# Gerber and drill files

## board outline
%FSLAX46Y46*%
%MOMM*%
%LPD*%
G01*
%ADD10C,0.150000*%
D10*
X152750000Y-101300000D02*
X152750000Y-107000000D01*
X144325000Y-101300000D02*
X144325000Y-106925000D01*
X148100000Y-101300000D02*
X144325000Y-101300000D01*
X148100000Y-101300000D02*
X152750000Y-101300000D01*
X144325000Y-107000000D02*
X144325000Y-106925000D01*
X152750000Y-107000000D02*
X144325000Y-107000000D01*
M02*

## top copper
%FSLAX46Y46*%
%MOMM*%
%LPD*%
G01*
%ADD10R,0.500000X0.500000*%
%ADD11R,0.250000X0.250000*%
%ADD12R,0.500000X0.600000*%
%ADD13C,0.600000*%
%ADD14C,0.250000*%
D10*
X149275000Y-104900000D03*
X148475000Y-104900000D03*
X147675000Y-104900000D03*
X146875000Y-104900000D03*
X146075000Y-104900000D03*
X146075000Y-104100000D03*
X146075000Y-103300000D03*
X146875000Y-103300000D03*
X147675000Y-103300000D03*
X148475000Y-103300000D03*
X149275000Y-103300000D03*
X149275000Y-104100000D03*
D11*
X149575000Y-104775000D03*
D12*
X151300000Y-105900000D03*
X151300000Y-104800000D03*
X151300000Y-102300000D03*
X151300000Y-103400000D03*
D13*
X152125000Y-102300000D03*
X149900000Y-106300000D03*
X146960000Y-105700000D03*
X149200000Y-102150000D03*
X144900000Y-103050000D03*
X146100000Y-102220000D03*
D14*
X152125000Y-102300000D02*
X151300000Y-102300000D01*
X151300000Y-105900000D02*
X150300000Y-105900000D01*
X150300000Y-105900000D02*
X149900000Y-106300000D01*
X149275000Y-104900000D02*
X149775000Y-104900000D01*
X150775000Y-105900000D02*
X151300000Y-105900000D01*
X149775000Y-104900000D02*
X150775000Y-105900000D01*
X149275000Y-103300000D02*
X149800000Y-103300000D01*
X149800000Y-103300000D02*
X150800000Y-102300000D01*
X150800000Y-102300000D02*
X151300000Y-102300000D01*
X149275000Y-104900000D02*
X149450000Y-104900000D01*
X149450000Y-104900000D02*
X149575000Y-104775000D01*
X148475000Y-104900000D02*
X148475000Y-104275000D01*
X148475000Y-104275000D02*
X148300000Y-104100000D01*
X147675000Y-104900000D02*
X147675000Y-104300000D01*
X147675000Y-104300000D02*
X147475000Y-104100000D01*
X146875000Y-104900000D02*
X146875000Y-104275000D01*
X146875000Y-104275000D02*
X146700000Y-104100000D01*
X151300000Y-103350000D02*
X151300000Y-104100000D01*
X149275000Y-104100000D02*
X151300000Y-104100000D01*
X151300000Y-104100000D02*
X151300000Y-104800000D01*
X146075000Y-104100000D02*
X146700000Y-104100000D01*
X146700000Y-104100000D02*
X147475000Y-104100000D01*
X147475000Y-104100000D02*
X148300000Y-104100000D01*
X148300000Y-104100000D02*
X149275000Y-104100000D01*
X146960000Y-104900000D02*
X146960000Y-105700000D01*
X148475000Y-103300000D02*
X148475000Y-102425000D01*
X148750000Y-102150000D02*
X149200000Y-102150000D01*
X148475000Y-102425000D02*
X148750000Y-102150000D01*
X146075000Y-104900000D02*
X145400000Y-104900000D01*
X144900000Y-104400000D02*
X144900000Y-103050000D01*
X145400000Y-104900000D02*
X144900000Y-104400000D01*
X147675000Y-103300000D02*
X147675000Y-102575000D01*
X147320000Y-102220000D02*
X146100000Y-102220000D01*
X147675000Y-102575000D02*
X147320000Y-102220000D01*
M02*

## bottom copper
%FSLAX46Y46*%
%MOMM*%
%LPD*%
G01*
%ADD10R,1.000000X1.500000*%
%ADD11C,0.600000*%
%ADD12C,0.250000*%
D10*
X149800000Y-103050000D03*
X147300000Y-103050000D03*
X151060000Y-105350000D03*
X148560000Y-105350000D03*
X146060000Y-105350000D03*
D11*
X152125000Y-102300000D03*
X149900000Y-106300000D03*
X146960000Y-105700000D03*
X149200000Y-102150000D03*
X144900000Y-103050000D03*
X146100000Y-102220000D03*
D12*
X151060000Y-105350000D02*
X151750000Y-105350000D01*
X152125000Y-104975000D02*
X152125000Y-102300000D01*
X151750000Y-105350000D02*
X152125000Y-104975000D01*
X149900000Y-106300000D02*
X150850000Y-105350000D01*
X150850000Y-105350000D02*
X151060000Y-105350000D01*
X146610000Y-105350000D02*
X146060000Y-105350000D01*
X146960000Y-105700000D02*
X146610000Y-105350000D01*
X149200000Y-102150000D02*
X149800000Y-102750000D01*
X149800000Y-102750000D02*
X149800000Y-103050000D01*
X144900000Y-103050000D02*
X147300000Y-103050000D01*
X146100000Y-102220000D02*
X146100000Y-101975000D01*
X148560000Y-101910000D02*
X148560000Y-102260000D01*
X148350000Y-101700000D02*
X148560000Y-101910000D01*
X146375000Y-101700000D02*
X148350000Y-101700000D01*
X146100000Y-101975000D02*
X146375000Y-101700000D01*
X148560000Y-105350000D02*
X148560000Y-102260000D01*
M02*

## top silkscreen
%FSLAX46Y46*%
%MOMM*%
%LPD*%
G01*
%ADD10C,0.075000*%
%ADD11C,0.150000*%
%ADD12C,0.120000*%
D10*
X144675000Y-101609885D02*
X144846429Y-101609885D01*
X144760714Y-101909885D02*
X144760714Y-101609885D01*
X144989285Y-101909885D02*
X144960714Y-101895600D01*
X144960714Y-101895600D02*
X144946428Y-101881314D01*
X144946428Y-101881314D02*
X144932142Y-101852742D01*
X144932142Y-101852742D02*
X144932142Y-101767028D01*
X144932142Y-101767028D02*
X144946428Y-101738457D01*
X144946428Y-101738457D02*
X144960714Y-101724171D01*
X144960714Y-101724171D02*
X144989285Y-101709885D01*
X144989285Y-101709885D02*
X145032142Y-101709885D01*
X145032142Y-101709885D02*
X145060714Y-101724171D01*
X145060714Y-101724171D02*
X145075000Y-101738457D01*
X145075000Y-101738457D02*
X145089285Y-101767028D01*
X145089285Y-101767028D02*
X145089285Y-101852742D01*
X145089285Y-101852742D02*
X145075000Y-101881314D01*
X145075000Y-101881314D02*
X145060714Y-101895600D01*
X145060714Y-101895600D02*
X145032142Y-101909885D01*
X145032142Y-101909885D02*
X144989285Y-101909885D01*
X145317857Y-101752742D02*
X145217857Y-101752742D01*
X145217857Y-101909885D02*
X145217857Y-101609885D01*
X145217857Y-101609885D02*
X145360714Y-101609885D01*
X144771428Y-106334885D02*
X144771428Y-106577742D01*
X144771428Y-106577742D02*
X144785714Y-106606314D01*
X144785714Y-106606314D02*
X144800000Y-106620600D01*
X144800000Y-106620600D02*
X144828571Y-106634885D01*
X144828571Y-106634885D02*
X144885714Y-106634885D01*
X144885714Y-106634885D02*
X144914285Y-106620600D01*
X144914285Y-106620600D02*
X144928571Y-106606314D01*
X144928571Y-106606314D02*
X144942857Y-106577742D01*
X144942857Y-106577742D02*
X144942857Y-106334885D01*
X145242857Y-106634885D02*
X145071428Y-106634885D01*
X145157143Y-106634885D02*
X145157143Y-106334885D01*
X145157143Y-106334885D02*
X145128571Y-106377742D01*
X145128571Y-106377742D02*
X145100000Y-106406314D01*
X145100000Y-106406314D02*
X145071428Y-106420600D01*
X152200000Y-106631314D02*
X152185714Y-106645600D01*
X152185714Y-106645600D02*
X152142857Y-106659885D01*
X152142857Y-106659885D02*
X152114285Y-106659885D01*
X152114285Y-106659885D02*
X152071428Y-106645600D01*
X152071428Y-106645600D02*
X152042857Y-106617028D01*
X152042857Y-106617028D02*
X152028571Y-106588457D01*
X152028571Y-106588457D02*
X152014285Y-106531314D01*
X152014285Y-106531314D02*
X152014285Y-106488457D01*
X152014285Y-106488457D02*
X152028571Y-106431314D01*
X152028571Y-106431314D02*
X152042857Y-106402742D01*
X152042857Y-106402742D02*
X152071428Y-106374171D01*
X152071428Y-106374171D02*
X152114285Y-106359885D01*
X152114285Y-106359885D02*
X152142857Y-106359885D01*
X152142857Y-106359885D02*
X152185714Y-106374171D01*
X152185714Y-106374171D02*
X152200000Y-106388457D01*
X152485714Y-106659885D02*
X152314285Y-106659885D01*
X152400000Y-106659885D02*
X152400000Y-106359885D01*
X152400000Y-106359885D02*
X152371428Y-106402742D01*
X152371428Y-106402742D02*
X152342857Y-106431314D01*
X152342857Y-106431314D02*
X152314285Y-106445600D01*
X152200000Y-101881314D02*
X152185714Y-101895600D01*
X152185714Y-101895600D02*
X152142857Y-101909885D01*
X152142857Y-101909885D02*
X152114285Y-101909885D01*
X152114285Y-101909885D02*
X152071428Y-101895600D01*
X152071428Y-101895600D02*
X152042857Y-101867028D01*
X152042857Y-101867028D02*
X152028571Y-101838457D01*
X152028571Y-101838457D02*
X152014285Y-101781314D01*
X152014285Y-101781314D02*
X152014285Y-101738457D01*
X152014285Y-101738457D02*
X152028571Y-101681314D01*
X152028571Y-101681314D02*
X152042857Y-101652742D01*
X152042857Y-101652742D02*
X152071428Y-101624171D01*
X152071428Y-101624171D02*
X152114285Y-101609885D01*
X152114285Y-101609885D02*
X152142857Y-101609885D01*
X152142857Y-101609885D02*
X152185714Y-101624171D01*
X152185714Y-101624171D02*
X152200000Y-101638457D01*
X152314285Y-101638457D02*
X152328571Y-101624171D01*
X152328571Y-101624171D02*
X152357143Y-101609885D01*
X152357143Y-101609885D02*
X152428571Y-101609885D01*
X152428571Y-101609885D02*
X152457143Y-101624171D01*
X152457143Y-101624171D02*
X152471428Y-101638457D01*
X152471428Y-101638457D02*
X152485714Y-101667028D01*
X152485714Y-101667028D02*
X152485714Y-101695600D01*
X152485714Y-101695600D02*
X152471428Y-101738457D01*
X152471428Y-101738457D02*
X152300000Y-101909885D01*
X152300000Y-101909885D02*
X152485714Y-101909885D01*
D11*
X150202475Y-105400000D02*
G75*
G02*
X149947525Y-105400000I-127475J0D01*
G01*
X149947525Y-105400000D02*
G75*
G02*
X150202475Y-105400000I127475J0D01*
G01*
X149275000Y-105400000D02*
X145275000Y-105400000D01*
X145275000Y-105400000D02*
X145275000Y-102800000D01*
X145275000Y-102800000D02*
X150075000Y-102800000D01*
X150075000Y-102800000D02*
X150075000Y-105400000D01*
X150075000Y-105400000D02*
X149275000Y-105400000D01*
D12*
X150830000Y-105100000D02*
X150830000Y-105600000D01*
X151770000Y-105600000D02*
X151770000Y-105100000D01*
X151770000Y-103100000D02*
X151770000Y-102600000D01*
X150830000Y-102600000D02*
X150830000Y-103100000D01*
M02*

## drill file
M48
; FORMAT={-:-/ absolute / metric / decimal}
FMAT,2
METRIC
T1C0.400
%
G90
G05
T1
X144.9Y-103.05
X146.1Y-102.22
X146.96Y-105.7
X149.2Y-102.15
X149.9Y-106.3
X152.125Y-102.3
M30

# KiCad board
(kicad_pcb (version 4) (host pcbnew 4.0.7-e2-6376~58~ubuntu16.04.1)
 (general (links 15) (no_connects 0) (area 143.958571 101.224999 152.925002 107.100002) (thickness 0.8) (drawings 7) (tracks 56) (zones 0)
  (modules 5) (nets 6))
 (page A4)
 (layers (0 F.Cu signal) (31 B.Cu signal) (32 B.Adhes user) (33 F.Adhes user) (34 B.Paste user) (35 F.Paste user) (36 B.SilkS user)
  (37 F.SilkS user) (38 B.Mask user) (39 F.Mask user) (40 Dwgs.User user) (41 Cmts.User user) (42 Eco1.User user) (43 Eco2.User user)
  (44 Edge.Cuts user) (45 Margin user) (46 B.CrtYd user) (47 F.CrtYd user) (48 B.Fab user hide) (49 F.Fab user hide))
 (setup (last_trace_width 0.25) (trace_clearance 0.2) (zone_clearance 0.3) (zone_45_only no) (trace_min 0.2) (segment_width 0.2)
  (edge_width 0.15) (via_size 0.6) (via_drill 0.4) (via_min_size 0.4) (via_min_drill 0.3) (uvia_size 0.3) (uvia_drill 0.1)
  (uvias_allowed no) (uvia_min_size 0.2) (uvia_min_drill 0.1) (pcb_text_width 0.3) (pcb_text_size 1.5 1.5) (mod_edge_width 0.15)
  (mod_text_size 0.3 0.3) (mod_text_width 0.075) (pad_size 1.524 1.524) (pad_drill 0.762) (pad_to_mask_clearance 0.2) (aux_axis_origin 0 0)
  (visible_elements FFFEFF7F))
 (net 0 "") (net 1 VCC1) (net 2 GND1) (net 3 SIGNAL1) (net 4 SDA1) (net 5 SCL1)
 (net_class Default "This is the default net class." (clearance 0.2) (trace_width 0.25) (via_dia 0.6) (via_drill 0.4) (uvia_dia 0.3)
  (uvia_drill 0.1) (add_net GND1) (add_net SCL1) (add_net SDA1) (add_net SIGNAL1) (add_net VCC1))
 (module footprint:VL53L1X (layer F.Cu) (at 149.275 104.9 90)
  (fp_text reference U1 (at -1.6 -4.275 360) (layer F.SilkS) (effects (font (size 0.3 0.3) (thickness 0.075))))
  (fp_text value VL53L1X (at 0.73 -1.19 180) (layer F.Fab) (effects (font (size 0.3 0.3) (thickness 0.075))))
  (fp_circle (center -0.5 0.8) (end -0.375 0.825) (layer F.SilkS) (width 0.15))
  (fp_line (start -0.5 0) (end -0.5 -4) (layer F.SilkS) (width 0.15))
  (fp_line (start -0.5 -4) (end 2.1 -4) (layer F.SilkS) (width 0.15))
  (fp_line (start 2.1 -4) (end 2.1 0.8) (layer F.SilkS) (width 0.15))
  (fp_line (start 2.1 0.8) (end -0.5 0.8) (layer F.SilkS) (width 0.15))
  (fp_line (start -0.5 0.8) (end -0.5 0) (layer F.SilkS) (width 0.15))
  (pad 1 smd rect (at 0 0 90) (size 0.5 0.5) (layers F.Cu F.Paste F.Mask) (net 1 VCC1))
  (pad 2 smd rect (at 0 -0.8 90) (size 0.5 0.5) (layers F.Cu F.Paste F.Mask) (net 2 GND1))
  (pad 3 smd rect (at 0 -1.6 90) (size 0.5 0.5) (layers F.Cu F.Paste F.Mask) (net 2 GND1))
  (pad 4 smd rect (at 0 -2.4 90) (size 0.5 0.5) (layers F.Cu F.Paste F.Mask) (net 2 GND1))
  (pad 5 smd rect (at 0 -3.2 90) (size 0.5 0.5) (layers F.Cu F.Paste F.Mask) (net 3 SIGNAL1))
  (pad 6 smd rect (at 0.8 -3.2 90) (size 0.5 0.5) (layers F.Cu F.Paste F.Mask) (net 2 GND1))
  (pad 7 smd rect (at 1.6 -3.2 90) (size 0.5 0.5) (layers F.Cu F.Paste F.Mask))
  (pad 8 smd rect (at 1.6 -2.4 90) (size 0.5 0.5) (layers F.Cu F.Paste F.Mask))
  (pad 9 smd rect (at 1.6 -1.6 90) (size 0.5 0.5) (layers F.Cu F.Paste F.Mask) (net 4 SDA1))
  (pad 10 smd rect (at 1.6 -0.8 90) (size 0.5 0.5) (layers F.Cu F.Paste F.Mask) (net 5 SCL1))
  (pad 11 smd rect (at 1.6 0 90) (size 0.5 0.5) (layers F.Cu F.Paste F.Mask) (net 1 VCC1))
  (pad 12 smd rect (at 0.8 0 90) (size 0.5 0.5) (layers F.Cu F.Paste F.Mask) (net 2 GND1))
  (pad 1 smd rect (at 0.125 0.3 90) (size 0.25 0.25) (layers F.Cu F.Paste F.Mask) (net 1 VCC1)))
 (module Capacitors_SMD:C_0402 (layer F.Cu) (at 151.3 105.35 90)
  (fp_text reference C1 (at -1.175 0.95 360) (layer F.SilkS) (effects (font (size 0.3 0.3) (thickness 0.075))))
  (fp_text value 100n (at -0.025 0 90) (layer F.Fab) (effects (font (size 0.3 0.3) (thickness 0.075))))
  (fp_line (start 0.25 -0.47) (end -0.25 -0.47) (layer F.SilkS) (width 0.12))
  (fp_line (start -0.25 0.47) (end 0.25 0.47) (layer F.SilkS) (width 0.12))
  (pad 1 smd rect (at -0.55 0 90) (size 0.6 0.5) (layers F.Cu F.Paste F.Mask) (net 1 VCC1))
  (pad 2 smd rect (at 0.55 0 90) (size 0.6 0.5) (layers F.Cu F.Paste F.Mask) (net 2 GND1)))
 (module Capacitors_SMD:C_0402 (layer F.Cu) (at 151.3 102.85 270)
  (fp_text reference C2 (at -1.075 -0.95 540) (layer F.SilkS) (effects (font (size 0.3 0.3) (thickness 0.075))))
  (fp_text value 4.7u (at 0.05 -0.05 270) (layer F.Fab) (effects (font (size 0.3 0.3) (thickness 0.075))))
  (fp_line (start 0.25 -0.47) (end -0.25 -0.47) (layer F.SilkS) (width 0.12))
  (fp_line (start -0.25 0.47) (end 0.25 0.47) (layer F.SilkS) (width 0.12))
  (pad 1 smd rect (at -0.55 0 270) (size 0.6 0.5) (layers F.Cu F.Paste F.Mask) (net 1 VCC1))
  (pad 2 smd rect (at 0.55 0 270) (size 0.6 0.5) (layers F.Cu F.Paste F.Mask) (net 2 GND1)))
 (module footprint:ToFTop (layer B.Cu) (at 148.55 103.3 180)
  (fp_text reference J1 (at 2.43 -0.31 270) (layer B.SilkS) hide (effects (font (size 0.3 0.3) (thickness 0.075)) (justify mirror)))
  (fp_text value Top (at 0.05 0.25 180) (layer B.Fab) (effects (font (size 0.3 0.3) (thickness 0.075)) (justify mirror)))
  (pad 1 smd rect (at -1.25 0.25 180) (size 1 1.5) (layers B.Cu B.Paste B.Mask) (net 5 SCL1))
  (pad 2 smd rect (at 1.25 0.25 180) (size 1 1.5) (layers B.Cu B.Paste B.Mask) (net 3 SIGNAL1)))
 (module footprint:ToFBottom (layer B.Cu) (at 148.56 105.1 180)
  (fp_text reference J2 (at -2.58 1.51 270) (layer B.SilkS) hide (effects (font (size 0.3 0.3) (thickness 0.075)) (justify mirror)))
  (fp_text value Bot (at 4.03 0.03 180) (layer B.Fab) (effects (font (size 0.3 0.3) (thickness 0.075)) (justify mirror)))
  (pad 1 smd rect (at -2.5 -0.25 180) (size 1 1.5) (layers B.Cu B.Paste B.Mask) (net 1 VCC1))
  (pad 2 smd rect (at 0 -0.25 180) (size 1 1.5) (layers B.Cu B.Paste B.Mask) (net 4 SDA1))
  (pad 3 smd rect (at 2.5 -0.25 180) (size 1 1.5) (layers B.Cu B.Paste B.Mask) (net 2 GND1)))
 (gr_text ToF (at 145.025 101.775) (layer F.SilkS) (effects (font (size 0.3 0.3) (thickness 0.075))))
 (gr_line (start 152.75 101.3) (end 152.75 107) (angle 90) (layer Edge.Cuts) (width 0.15))
 (gr_line (start 144.325 101.3) (end 144.325 106.925) (angle 90) (layer Edge.Cuts) (width 0.15))
 (gr_line (start 148.1 101.3) (end 144.325 101.3) (angle 90) (layer Edge.Cuts) (width 0.15))
 (gr_line (start 148.1 101.3) (end 152.75 101.3) (angle 90) (layer Edge.Cuts) (width 0.15))
 (gr_line (start 144.325 107) (end 144.325 106.925) (angle 90) (layer Edge.Cuts) (width 0.15))
 (gr_line (start 152.75 107) (end 144.325 107) (angle 90) (layer Edge.Cuts) (width 0.15))
 (segment (start 151.06 105.35) (end 151.75 105.35) (width 0.25) (layer B.Cu) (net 1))
 (segment (start 152.125 102.3) (end 151.3 102.3) (width 0.25) (layer F.Cu) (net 1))
 (via (at 152.125 102.3) (size 0.6) (drill 0.4) (layers F.Cu B.Cu) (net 1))
 (segment (start 152.125 104.975) (end 152.125 102.3) (width 0.25) (layer B.Cu) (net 1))
 (segment (start 151.75 105.35) (end 152.125 104.975) (width 0.25) (layer B.Cu) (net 1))
 (segment (start 151.3 105.9) (end 150.3 105.9) (width 0.25) (layer F.Cu) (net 1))
 (segment (start 149.9 106.3) (end 150.85 105.35) (width 0.25) (layer B.Cu) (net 1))
 (via (at 149.9 106.3) (size 0.6) (drill 0.4) (layers F.Cu B.Cu) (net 1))
 (segment (start 150.3 105.9) (end 149.9 106.3) (width 0.25) (layer F.Cu) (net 1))
 (segment (start 150.85 105.35) (end 151.06 105.35) (width 0.25) (layer B.Cu) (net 1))
 (segment (start 149.275 104.9) (end 149.775 104.9) (width 0.25) (layer F.Cu) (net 1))
 (segment (start 150.775 105.9) (end 151.3 105.9) (width 0.25) (layer F.Cu) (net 1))
 (segment (start 149.775 104.9) (end 150.775 105.9) (width 0.25) (layer F.Cu) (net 1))
 (segment (start 149.275 103.3) (end 149.8 103.3) (width 0.25) (layer F.Cu) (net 1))
 (segment (start 149.8 103.3) (end 150.8 102.3) (width 0.25) (layer F.Cu) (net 1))
 (segment (start 150.8 102.3) (end 151.3 102.3) (width 0.25) (layer F.Cu) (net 1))
 (segment (start 149.275 104.9) (end 149.45 104.9) (width 0.25) (layer F.Cu) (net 1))
 (segment (start 149.45 104.9) (end 149.575 104.775) (width 0.25) (layer F.Cu) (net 1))
 (segment (start 148.475 104.9) (end 148.475 104.275) (width 0.25) (layer F.Cu) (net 2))
 (segment (start 148.475 104.275) (end 148.3 104.1) (width 0.25) (layer F.Cu) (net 2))
 (segment (start 147.675 104.9) (end 147.675 104.3) (width 0.25) (layer F.Cu) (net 2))
 (segment (start 147.675 104.3) (end 147.475 104.1) (width 0.25) (layer F.Cu) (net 2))
 (segment (start 146.875 104.9) (end 146.875 104.275) (width 0.25) (layer F.Cu) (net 2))
 (segment (start 146.875 104.275) (end 146.7 104.1) (width 0.25) (layer F.Cu) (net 2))
 (segment (start 151.3 103.35) (end 151.3 104.1) (width 0.25) (layer F.Cu) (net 2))
 (segment (start 149.275 104.1) (end 151.3 104.1) (width 0.25) (layer F.Cu) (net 2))
 (segment (start 151.3 104.1) (end 151.3 104.8) (width 0.25) (layer F.Cu) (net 2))
 (segment (start 146.075 104.1) (end 146.7 104.1) (width 0.25) (layer F.Cu) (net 2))
 (segment (start 146.7 104.1) (end 147.475 104.1) (width 0.25) (layer F.Cu) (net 2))
 (segment (start 147.475 104.1) (end 148.3 104.1) (width 0.25) (layer F.Cu) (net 2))
 (segment (start 148.3 104.1) (end 149.275 104.1) (width 0.25) (layer F.Cu) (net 2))
 (segment (start 146.96 104.9) (end 146.96 105.7) (width 0.25) (layer F.Cu) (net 2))
 (segment (start 146.61 105.35) (end 146.06 105.35) (width 0.25) (layer B.Cu) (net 2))
 (segment (start 146.96 105.7) (end 146.61 105.35) (width 0.25) (layer B.Cu) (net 2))
 (via (at 146.96 105.7) (size 0.6) (drill 0.4) (layers F.Cu B.Cu) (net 2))
 (segment (start 148.475 103.3) (end 148.475 102.425) (width 0.25) (layer F.Cu) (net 5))
 (segment (start 148.75 102.15) (end 149.2 102.15) (width 0.25) (layer F.Cu) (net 5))
 (segment (start 148.475 102.425) (end 148.75 102.15) (width 0.25) (layer F.Cu) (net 5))
 (segment (start 149.2 102.15) (end 149.8 102.75) (width 0.25) (layer B.Cu) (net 5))
 (via (at 149.2 102.15) (size 0.6) (drill 0.4) (layers F.Cu B.Cu) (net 5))
 (segment (start 149.8 102.75) (end 149.8 103.05) (width 0.25) (layer B.Cu) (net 5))
 (segment (start 146.075 104.9) (end 145.4 104.9) (width 0.25) (layer F.Cu) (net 3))
 (segment (start 144.9 103.05) (end 147.3 103.05) (width 0.25) (layer B.Cu) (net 3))
 (via (at 144.9 103.05) (size 0.6) (drill 0.4) (layers F.Cu B.Cu) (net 3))
 (segment (start 144.9 104.4) (end 144.9 103.05) (width 0.25) (layer F.Cu) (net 3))
 (segment (start 145.4 104.9) (end 144.9 104.4) (width 0.25) (layer F.Cu) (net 3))
 (segment (start 146.1 102.22) (end 146.1 101.975) (width 0.25) (layer B.Cu) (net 4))
 (segment (start 148.56 101.91) (end 148.56 102.26) (width 0.25) (layer B.Cu) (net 4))
 (segment (start 148.35 101.7) (end 148.56 101.91) (width 0.25) (layer B.Cu) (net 4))
 (segment (start 146.375 101.7) (end 148.35 101.7) (width 0.25) (layer B.Cu) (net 4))
 (segment (start 146.1 101.975) (end 146.375 101.7) (width 0.25) (layer B.Cu) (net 4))
 (segment (start 147.675 103.3) (end 147.675 102.575) (width 0.25) (layer F.Cu) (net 4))
 (segment (start 147.32 102.22) (end 146.1 102.22) (width 0.25) (layer F.Cu) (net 4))
 (segment (start 147.675 102.575) (end 147.32 102.22) (width 0.25) (layer F.Cu) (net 4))
 (segment (start 148.56 105.35) (end 148.56 102.26) (width 0.25) (layer B.Cu) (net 4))
 (via (at 146.1 102.22) (size 0.6) (drill 0.4) (layers F.Cu B.Cu) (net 4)))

